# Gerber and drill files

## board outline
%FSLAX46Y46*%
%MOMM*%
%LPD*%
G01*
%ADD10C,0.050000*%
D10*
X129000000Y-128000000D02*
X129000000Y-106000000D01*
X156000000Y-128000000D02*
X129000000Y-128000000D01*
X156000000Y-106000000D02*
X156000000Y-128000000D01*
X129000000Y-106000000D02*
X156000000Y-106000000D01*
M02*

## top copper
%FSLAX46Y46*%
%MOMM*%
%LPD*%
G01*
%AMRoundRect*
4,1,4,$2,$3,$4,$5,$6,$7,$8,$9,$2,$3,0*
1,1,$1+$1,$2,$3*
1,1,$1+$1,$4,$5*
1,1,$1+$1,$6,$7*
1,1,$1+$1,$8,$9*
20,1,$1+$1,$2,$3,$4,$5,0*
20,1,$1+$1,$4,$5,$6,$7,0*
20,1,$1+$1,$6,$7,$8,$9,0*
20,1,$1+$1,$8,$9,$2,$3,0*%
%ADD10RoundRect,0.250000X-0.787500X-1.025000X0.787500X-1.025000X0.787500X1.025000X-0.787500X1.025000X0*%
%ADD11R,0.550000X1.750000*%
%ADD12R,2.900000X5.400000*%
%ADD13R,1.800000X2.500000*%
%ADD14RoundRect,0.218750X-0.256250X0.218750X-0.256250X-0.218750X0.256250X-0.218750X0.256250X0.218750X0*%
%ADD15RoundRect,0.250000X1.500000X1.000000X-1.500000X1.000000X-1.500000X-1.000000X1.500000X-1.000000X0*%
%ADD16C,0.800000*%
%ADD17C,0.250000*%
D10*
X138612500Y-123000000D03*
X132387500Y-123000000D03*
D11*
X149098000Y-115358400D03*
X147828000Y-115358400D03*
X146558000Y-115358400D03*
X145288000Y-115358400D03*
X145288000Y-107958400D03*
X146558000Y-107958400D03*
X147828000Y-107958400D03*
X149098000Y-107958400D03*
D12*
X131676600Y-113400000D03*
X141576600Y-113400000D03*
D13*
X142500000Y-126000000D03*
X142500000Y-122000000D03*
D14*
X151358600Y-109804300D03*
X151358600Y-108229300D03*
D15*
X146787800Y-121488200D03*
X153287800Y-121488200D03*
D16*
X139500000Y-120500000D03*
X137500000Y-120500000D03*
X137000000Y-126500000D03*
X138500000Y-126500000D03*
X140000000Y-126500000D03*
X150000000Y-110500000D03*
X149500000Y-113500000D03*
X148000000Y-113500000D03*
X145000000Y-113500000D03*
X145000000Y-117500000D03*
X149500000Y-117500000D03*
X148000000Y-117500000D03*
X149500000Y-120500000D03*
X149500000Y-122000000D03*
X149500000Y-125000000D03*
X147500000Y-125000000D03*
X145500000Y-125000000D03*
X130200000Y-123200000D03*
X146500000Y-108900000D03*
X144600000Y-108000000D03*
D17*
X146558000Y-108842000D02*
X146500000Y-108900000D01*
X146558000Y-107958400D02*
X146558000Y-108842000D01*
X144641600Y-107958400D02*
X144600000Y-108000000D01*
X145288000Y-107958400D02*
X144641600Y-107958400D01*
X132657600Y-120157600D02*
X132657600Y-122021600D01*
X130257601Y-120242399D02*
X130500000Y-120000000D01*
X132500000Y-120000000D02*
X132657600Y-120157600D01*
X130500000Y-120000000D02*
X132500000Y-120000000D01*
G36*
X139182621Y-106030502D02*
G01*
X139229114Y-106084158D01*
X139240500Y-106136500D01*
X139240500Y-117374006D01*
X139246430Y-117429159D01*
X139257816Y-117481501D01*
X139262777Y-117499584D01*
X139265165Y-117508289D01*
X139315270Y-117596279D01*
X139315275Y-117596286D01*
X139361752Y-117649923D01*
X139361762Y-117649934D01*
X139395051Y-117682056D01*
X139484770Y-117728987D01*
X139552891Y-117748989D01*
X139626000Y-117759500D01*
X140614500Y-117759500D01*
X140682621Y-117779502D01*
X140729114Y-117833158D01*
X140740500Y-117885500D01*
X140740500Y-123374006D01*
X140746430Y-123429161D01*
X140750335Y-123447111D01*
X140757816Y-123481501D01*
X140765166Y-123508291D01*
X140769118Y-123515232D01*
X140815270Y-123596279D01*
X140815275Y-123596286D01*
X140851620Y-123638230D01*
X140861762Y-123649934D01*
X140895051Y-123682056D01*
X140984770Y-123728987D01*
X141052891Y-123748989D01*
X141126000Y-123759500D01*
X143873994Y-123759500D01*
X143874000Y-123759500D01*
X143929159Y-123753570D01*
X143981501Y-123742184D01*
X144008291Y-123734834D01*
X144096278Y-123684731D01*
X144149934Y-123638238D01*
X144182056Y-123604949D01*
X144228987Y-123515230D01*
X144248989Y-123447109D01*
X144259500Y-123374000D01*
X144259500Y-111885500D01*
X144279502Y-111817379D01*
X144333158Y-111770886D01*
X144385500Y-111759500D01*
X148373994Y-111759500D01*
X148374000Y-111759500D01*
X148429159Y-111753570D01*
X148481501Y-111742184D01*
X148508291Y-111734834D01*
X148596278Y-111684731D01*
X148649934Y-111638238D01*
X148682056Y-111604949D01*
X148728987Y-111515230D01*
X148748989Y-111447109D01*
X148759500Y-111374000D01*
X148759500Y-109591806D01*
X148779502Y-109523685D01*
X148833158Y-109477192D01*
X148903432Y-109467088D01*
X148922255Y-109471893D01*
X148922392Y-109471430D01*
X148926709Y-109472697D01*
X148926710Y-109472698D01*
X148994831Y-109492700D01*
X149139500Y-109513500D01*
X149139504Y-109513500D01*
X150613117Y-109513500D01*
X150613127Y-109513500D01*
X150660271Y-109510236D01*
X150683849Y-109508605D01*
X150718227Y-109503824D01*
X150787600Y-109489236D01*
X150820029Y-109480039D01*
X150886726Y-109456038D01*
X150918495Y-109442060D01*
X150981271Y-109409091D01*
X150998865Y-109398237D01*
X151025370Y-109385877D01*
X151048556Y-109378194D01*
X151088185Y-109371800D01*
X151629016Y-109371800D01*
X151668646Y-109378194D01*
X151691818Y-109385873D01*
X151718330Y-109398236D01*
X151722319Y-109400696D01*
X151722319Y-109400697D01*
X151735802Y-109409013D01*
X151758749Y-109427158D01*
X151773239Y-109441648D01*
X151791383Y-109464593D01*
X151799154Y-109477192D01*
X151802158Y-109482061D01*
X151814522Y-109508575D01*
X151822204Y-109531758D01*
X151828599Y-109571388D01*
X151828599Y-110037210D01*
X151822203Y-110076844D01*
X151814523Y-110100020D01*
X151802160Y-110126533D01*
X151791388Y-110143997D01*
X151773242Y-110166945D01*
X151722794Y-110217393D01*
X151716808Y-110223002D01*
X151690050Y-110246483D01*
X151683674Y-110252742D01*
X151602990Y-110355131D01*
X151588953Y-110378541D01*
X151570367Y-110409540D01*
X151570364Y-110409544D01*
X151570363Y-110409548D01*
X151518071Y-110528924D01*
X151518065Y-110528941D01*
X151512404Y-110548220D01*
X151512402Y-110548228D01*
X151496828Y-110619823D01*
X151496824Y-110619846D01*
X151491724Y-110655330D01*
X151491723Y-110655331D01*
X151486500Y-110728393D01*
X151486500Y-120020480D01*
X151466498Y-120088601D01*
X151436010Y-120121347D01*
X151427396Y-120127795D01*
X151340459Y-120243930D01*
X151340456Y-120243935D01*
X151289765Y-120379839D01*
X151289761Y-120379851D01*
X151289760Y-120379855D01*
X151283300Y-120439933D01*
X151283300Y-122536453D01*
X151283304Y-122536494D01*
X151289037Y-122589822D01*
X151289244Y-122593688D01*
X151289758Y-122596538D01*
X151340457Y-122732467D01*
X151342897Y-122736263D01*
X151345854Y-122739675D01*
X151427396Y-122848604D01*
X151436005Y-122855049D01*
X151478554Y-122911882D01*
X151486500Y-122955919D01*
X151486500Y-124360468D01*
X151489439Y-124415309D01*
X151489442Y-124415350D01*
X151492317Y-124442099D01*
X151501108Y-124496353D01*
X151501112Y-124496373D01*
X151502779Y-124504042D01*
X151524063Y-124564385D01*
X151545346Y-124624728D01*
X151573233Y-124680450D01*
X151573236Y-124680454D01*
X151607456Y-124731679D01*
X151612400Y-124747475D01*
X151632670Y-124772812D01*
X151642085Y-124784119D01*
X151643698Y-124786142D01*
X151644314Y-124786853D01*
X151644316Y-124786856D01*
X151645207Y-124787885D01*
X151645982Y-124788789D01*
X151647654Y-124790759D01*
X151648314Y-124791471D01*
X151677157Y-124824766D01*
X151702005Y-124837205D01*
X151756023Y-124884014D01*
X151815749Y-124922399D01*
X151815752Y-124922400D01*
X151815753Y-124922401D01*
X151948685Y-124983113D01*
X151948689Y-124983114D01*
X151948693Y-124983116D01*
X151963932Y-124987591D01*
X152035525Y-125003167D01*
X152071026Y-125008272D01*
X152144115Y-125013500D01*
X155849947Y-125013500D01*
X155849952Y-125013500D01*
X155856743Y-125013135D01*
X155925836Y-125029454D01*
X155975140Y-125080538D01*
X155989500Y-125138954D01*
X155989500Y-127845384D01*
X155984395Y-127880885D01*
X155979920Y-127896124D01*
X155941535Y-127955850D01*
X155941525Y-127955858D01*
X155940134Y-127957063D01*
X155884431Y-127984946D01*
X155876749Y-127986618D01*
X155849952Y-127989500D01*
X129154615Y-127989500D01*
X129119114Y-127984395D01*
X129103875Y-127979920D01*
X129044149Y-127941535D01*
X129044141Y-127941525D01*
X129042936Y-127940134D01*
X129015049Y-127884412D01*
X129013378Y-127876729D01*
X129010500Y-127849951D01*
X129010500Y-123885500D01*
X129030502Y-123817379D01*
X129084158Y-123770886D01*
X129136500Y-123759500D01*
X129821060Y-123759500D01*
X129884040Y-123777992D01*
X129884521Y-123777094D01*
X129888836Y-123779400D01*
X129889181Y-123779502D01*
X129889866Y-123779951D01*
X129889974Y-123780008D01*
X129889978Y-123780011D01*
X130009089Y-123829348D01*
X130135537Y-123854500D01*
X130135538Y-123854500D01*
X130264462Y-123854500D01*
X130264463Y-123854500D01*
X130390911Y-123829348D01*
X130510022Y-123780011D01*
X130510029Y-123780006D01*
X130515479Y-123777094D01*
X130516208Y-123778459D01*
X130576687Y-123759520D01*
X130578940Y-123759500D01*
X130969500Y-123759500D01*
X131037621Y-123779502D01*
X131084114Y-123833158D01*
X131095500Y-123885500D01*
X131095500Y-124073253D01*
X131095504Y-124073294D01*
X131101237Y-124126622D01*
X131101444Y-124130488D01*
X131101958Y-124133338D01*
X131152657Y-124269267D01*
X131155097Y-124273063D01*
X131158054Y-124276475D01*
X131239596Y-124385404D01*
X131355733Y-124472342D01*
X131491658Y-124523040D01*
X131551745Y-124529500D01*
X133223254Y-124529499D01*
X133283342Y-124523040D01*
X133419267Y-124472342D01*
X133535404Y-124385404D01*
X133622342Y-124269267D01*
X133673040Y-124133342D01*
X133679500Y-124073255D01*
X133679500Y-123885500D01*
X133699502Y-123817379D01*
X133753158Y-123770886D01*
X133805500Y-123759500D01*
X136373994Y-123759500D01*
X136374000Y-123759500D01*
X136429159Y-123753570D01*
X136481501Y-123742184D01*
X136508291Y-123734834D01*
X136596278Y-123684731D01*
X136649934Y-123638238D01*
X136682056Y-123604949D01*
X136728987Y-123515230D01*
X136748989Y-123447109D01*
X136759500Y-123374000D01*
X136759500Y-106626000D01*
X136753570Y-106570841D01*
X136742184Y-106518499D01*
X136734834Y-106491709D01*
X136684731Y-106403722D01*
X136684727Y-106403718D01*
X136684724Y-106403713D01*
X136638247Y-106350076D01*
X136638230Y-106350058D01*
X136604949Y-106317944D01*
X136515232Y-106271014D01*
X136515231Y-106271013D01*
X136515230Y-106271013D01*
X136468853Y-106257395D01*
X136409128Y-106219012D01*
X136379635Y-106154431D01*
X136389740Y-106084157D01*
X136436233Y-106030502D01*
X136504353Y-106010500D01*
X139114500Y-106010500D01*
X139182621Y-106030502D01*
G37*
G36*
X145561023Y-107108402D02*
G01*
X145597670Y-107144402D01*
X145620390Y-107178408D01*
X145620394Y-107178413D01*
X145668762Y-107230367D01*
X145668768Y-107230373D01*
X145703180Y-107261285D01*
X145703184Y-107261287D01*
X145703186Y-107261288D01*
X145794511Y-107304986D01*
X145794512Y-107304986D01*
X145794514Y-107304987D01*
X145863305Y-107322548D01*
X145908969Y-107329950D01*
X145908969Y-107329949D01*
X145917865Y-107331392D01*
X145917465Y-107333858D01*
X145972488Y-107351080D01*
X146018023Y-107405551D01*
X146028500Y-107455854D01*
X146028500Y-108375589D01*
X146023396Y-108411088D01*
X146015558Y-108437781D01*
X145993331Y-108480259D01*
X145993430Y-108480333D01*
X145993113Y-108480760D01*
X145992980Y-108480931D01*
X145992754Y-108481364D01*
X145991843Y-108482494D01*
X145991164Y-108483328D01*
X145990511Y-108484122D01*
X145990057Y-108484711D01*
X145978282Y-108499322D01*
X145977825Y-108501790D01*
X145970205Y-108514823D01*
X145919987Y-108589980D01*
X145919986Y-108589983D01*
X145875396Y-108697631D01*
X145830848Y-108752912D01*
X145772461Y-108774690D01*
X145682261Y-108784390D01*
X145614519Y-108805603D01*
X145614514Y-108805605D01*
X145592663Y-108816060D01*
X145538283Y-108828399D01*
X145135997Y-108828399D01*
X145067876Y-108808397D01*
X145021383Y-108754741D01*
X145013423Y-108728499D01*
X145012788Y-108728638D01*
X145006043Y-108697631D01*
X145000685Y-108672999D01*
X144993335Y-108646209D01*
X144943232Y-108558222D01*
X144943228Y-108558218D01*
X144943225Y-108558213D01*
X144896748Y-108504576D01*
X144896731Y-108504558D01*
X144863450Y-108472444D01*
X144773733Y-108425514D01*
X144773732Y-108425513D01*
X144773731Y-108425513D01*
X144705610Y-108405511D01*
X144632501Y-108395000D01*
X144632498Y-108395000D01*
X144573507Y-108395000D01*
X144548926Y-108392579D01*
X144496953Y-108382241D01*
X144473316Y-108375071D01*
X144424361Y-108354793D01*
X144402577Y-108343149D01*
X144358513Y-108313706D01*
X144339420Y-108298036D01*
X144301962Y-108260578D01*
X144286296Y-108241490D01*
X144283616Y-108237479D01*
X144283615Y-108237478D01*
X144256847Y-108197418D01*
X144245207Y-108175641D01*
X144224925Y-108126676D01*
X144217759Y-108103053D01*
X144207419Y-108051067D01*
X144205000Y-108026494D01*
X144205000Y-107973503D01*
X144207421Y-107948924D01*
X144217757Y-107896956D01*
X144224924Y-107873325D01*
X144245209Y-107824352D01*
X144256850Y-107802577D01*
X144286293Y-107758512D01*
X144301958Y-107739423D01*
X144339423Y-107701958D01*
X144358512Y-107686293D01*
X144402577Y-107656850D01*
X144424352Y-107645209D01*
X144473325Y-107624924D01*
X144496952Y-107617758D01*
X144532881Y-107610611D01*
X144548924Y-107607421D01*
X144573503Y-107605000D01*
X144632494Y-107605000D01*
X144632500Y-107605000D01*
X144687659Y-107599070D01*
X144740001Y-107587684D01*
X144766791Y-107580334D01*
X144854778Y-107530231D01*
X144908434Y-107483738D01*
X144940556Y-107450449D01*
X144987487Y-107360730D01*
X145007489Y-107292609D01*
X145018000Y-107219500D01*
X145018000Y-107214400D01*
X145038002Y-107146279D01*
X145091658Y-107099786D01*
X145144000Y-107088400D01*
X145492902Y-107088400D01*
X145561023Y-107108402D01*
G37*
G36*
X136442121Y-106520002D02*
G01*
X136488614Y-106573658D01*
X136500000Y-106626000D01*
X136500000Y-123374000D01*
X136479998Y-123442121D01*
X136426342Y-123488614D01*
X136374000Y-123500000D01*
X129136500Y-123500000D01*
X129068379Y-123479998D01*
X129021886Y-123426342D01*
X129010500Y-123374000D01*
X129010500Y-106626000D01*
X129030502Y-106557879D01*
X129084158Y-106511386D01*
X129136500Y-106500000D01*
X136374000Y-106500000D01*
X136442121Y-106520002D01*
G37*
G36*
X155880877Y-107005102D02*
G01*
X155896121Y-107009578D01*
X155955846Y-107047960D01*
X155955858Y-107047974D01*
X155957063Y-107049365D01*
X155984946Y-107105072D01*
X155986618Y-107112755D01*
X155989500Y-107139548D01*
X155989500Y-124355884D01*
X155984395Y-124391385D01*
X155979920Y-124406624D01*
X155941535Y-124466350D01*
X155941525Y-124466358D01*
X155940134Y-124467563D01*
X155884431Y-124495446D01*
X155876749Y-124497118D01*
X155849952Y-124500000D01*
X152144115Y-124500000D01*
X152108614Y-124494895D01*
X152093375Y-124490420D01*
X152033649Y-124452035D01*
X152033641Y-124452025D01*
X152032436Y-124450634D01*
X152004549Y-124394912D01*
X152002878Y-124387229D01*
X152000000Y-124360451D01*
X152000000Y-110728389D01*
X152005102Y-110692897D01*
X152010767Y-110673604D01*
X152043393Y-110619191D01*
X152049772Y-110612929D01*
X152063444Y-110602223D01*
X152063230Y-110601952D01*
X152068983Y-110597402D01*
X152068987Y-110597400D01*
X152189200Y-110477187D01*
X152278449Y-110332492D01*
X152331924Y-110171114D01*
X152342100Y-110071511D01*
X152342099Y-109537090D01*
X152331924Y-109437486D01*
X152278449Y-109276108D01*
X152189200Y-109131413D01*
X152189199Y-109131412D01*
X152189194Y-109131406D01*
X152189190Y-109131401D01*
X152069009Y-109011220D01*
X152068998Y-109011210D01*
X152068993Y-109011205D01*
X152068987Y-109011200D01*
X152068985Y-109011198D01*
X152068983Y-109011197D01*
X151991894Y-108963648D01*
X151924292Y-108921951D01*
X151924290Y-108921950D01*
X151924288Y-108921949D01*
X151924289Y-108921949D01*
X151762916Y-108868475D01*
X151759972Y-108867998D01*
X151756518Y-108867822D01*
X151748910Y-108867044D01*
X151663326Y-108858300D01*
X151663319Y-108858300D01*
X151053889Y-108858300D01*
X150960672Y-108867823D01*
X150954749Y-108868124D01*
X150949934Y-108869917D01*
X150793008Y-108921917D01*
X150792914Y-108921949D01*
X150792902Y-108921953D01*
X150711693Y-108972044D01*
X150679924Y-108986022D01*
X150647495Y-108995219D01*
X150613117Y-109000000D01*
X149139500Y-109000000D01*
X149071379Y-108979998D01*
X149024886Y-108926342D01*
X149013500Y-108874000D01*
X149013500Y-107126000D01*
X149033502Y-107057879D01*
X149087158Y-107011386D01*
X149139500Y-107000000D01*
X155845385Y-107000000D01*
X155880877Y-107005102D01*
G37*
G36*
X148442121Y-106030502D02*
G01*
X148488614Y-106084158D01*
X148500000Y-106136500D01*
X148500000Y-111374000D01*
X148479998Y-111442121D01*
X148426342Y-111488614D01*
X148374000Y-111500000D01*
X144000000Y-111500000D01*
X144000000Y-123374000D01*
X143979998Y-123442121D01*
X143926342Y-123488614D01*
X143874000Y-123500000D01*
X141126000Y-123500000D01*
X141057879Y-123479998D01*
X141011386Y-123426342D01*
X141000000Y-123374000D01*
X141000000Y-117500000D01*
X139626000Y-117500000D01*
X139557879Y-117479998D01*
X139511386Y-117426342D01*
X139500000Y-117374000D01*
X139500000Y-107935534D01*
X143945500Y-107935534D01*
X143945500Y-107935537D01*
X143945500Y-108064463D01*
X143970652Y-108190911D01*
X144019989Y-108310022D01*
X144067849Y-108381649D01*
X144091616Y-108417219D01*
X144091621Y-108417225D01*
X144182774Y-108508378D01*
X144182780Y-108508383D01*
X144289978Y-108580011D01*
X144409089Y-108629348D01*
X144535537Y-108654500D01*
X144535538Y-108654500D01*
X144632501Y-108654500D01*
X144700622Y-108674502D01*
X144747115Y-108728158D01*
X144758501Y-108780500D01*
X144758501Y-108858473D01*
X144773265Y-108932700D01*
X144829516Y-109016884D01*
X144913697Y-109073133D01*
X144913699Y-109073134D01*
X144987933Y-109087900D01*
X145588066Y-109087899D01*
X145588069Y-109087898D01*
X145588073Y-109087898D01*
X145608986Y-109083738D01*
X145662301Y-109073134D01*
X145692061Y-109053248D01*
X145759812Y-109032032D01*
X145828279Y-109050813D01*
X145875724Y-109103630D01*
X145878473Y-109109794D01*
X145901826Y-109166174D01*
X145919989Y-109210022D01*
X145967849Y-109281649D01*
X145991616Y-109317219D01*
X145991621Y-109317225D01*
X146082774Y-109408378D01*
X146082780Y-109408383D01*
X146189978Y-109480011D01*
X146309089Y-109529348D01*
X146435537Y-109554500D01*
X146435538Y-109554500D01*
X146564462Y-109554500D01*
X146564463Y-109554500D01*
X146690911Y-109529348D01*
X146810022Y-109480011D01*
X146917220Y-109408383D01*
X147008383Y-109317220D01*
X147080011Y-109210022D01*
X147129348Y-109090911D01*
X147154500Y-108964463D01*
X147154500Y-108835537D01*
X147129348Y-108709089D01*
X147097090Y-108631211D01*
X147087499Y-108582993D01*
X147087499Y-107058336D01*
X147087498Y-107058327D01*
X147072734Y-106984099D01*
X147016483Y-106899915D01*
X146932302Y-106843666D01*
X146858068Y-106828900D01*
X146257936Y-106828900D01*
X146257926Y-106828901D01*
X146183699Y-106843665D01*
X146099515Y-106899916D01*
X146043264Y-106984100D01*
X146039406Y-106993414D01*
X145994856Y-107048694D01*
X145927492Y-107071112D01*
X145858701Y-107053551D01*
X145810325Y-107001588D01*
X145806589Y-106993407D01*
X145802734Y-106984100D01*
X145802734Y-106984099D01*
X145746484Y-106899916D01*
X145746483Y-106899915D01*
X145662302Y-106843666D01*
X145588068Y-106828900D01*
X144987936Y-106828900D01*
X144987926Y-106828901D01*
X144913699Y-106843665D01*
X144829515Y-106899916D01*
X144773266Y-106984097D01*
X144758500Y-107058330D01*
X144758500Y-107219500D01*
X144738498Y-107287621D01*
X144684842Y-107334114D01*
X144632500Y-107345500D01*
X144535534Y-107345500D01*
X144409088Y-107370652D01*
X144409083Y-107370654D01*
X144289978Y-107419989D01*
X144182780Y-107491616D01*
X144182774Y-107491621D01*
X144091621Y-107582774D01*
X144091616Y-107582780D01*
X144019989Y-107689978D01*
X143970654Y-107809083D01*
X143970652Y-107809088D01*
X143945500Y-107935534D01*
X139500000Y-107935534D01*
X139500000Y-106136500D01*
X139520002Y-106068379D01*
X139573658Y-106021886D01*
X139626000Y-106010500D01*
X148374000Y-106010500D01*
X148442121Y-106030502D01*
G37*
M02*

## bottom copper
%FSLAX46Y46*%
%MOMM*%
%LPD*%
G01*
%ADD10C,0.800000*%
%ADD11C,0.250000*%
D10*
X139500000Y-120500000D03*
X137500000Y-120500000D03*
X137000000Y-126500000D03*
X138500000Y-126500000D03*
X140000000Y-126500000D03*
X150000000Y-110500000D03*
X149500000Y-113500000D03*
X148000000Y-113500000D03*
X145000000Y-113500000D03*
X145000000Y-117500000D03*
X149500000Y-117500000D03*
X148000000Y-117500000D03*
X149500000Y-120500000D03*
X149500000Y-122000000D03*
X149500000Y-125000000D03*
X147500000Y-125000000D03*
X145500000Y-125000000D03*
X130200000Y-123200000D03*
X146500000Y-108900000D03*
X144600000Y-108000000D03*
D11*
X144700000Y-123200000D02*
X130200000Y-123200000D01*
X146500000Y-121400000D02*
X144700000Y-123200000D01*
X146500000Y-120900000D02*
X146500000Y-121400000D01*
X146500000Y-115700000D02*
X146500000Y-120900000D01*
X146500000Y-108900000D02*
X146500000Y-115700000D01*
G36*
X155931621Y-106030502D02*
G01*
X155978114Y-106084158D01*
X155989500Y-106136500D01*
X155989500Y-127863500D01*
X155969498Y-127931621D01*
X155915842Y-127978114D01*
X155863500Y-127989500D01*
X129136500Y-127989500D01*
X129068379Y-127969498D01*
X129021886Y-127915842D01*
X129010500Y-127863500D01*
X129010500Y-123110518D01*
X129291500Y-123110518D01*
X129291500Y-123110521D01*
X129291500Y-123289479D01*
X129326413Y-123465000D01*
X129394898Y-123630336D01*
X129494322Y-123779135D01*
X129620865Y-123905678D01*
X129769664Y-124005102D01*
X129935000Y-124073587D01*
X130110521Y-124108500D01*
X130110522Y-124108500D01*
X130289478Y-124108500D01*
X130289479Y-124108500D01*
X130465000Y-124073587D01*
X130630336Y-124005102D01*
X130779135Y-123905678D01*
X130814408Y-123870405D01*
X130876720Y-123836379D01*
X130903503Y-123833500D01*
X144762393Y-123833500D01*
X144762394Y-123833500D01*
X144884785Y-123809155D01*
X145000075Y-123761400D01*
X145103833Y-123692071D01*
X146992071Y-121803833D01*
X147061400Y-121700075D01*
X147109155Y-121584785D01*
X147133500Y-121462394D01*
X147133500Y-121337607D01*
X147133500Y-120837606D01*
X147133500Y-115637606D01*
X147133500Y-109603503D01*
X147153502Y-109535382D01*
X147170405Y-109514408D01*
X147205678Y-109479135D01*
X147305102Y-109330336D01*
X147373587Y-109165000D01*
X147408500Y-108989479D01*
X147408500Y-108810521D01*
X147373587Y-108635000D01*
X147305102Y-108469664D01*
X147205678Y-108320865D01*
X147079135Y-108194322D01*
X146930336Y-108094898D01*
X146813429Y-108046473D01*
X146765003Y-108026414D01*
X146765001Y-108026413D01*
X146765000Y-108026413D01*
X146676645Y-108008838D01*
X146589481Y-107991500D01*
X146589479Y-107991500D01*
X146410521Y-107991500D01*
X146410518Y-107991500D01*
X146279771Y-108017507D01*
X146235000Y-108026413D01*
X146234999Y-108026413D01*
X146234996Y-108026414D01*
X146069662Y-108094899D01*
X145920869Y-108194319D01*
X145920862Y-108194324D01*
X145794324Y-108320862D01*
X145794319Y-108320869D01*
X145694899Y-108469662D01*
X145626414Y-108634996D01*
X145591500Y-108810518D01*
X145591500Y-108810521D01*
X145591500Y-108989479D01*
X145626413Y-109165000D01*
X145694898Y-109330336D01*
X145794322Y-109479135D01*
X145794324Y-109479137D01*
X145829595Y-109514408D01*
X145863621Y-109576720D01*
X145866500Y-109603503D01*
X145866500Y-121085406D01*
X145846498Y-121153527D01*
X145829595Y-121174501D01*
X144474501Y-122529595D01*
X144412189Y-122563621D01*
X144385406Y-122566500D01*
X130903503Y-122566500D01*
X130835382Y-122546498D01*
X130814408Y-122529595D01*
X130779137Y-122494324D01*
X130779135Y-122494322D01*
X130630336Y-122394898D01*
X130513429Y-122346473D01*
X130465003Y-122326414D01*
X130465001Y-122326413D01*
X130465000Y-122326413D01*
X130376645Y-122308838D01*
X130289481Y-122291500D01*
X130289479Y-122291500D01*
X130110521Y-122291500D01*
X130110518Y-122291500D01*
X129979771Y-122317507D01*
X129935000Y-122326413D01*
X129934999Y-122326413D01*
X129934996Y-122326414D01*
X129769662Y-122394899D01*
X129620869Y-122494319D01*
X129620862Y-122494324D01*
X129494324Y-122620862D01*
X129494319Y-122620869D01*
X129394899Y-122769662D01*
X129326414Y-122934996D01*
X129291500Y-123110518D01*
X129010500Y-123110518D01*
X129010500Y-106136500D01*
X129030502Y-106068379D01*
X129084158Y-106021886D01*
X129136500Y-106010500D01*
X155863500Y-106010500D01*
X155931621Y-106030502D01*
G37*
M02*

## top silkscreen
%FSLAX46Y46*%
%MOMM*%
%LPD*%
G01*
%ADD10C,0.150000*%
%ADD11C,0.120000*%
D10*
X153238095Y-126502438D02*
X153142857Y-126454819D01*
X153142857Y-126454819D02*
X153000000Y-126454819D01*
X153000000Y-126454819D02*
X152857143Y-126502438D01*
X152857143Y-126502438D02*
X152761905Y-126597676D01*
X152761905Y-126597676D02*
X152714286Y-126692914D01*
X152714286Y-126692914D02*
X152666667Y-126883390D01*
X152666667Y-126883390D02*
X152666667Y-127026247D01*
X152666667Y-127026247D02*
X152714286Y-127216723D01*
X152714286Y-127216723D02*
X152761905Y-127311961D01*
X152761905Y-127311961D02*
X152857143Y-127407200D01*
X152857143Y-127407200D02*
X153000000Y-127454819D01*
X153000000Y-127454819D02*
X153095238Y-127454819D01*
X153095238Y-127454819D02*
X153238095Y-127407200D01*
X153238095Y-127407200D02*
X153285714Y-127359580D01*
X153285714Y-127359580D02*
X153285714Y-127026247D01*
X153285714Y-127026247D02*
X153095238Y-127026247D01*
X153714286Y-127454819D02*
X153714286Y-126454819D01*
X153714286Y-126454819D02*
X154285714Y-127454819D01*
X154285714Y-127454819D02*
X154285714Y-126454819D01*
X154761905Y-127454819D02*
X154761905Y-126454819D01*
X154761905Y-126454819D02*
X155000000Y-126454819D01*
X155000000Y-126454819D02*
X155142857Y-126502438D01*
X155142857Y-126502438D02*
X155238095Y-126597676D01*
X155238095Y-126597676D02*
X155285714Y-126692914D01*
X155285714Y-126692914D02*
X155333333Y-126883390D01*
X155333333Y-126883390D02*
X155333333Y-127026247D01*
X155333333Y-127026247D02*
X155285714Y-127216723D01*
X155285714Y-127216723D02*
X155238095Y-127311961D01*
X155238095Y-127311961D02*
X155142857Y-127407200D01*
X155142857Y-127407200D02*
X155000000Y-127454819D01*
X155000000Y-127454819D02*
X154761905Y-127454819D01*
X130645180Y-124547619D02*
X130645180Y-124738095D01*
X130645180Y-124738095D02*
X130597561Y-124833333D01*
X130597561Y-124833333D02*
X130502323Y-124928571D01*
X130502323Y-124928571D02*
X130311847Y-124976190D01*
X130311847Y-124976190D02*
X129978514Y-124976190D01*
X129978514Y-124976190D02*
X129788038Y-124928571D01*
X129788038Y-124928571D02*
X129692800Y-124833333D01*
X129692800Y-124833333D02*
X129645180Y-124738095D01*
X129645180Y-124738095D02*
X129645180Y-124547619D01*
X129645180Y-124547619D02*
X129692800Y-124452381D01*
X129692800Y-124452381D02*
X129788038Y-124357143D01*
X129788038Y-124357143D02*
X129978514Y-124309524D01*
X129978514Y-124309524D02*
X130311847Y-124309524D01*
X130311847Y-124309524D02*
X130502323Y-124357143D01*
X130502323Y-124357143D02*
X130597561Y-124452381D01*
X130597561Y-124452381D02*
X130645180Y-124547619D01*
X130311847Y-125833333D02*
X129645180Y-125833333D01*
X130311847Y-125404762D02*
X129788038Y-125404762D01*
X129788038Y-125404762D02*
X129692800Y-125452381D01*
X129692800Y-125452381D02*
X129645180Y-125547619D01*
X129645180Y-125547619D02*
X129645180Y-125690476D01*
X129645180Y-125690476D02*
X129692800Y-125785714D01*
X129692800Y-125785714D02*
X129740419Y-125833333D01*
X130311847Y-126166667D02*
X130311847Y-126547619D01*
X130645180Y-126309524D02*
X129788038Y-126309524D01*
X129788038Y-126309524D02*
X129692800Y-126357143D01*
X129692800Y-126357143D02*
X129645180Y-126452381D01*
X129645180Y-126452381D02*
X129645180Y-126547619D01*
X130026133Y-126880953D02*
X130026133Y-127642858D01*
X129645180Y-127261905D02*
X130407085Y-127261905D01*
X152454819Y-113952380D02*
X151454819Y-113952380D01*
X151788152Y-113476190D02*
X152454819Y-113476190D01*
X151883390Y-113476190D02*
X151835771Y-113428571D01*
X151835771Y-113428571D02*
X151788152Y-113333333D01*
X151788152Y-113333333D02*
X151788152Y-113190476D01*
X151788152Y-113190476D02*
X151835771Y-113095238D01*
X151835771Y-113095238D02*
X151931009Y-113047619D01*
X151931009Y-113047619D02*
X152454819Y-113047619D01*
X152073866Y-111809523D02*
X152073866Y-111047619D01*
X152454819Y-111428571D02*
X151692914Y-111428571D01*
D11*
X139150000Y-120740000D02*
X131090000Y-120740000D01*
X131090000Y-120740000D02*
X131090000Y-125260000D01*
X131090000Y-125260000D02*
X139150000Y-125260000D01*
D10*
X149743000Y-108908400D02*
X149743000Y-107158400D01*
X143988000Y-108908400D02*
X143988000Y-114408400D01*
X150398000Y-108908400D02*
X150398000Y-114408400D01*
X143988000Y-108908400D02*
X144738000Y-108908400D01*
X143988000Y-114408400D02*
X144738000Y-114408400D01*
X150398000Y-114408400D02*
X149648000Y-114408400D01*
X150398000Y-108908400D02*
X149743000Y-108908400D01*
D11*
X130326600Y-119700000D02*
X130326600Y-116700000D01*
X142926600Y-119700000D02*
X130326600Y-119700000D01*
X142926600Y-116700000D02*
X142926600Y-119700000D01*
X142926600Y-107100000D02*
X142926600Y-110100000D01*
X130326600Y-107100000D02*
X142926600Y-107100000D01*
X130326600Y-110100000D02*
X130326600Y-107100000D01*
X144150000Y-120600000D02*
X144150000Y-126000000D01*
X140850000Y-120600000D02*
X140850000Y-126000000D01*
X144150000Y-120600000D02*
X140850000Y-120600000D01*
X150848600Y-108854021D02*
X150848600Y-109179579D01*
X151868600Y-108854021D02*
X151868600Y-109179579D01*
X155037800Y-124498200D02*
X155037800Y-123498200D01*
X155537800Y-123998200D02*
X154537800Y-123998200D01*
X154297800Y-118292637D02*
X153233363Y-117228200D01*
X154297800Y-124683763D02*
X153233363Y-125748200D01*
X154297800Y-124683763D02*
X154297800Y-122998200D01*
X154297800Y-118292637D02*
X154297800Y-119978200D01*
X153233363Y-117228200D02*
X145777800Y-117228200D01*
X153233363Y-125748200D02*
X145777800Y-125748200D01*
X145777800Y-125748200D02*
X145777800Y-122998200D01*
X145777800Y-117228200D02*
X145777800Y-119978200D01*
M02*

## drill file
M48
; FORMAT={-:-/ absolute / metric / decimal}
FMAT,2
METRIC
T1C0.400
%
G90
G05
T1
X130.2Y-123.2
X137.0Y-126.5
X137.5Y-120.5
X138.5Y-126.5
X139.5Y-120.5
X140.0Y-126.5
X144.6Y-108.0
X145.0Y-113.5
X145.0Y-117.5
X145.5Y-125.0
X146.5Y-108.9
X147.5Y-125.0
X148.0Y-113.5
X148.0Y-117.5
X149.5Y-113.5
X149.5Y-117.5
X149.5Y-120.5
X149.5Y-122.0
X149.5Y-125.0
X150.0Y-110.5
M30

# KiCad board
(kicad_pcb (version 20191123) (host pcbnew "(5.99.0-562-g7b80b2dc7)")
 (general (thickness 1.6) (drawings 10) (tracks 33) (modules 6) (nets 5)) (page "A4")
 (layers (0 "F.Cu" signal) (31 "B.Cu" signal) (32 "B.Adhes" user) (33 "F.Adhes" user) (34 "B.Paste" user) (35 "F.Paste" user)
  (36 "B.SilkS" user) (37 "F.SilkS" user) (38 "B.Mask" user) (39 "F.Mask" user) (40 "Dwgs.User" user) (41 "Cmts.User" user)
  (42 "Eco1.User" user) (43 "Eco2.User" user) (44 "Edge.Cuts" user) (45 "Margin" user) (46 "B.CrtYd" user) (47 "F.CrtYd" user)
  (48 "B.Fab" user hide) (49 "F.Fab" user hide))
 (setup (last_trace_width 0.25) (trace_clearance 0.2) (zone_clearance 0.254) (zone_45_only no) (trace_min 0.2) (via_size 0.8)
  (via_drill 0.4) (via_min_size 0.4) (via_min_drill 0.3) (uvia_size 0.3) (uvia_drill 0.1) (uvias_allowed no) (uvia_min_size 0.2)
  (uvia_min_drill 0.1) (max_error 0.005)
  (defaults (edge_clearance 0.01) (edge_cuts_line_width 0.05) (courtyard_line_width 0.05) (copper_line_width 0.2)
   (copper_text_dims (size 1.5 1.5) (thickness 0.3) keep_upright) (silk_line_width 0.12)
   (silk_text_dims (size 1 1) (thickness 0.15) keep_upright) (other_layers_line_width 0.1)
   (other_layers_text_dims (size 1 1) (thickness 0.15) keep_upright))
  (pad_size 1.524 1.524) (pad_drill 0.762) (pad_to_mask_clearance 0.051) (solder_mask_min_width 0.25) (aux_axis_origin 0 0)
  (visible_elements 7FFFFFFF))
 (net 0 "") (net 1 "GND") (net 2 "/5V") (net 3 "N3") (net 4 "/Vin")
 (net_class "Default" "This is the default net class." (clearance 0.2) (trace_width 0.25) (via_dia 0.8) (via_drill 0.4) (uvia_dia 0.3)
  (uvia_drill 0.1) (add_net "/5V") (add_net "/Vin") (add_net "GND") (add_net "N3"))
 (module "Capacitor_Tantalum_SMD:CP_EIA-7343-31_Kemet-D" (layer "F.Cu") (at 135.5 123)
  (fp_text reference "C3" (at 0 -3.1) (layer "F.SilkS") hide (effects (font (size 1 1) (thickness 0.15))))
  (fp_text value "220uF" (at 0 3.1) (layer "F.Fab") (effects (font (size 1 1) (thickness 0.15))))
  (fp_line (start 3.65 -2.26) (end -4.41 -2.26) (layer "F.SilkS") (width 0.12))
  (fp_line (start -4.41 -2.26) (end -4.41 2.26) (layer "F.SilkS") (width 0.12))
  (fp_line (start -4.41 2.26) (end 3.65 2.26) (layer "F.SilkS") (width 0.12))
  (pad "2" smd roundrect (at 3.1125 0) (size 2.075 2.55) (layers "F.Cu" "F.Paste" "F.Mask") (roundrect_rratio 0.120482) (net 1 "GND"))
  (pad "1" smd roundrect (at -3.1125 0) (size 2.075 2.55) (layers "F.Cu" "F.Paste" "F.Mask") (roundrect_rratio 0.120482) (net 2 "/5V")))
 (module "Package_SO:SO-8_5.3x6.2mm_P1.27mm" (layer "F.Cu") (at 147.193 111.6584 -90)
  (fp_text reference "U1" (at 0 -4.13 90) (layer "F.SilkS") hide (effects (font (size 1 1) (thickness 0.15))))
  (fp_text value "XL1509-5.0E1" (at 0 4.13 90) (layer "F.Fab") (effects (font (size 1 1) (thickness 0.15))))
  (fp_line (start -2.75 -2.55) (end -4.5 -2.55) (layer "F.SilkS") (width 0.15))
  (fp_line (start -2.75 3.205) (end 2.75 3.205) (layer "F.SilkS") (width 0.15))
  (fp_line (start -2.75 -3.205) (end 2.75 -3.205) (layer "F.SilkS") (width 0.15))
  (fp_line (start -2.75 3.205) (end -2.75 2.455) (layer "F.SilkS") (width 0.15))
  (fp_line (start 2.75 3.205) (end 2.75 2.455) (layer "F.SilkS") (width 0.15))
  (fp_line (start 2.75 -3.205) (end 2.75 -2.455) (layer "F.SilkS") (width 0.15))
  (fp_line (start -2.75 -3.205) (end -2.75 -2.55) (layer "F.SilkS") (width 0.15))
  (pad "8" smd rect (at 3.7 -1.905 270) (size 1.75 0.55) (layers "F.Cu" "F.Paste" "F.Mask") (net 1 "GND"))
  (pad "7" smd rect (at 3.7 -0.635 270) (size 1.75 0.55) (layers "F.Cu" "F.Paste" "F.Mask") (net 1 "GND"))
  (pad "6" smd rect (at 3.7 0.635 270) (size 1.75 0.55) (layers "F.Cu" "F.Paste" "F.Mask") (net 1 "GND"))
  (pad "5" smd rect (at 3.7 1.905 270) (size 1.75 0.55) (layers "F.Cu" "F.Paste" "F.Mask") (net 1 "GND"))
  (pad "4" smd rect (at -3.7 1.905 270) (size 1.75 0.55) (layers "F.Cu" "F.Paste" "F.Mask") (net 1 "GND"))
  (pad "3" smd rect (at -3.7 0.635 270) (size 1.75 0.55) (layers "F.Cu" "F.Paste" "F.Mask") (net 2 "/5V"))
  (pad "2" smd rect (at -3.7 -0.635 270) (size 1.75 0.55) (layers "F.Cu" "F.Paste" "F.Mask") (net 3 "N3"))
  (pad "1" smd rect (at -3.7 -1.905 270) (size 1.75 0.55) (layers "F.Cu" "F.Paste" "F.Mask") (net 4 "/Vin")))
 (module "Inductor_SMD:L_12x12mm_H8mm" (layer "F.Cu") (at 136.6266 113.4 180)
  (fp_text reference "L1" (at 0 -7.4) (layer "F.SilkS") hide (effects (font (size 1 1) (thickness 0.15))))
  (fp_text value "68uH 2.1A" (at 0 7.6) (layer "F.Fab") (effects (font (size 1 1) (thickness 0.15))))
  (fp_line (start 6.3 -6.3) (end 6.3 -3.3) (layer "F.SilkS") (width 0.12))
  (fp_line (start -6.3 -6.3) (end 6.3 -6.3) (layer "F.SilkS") (width 0.12))
  (fp_line (start -6.3 -3.3) (end -6.3 -6.3) (layer "F.SilkS") (width 0.12))
  (fp_line (start -6.3 6.3) (end -6.3 3.3) (layer "F.SilkS") (width 0.12))
  (fp_line (start 6.3 6.3) (end -6.3 6.3) (layer "F.SilkS") (width 0.12))
  (fp_line (start 6.3 3.3) (end 6.3 6.3) (layer "F.SilkS") (width 0.12))
  (pad "2" smd rect (at 4.95 0 180) (size 2.9 5.4) (layers "F.Cu" "F.Paste" "F.Mask") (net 2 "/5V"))
  (pad "1" smd rect (at -4.95 0 180) (size 2.9 5.4) (layers "F.Cu" "F.Paste" "F.Mask") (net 3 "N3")))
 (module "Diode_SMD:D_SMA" (layer "F.Cu") (at 142.5 124 -90)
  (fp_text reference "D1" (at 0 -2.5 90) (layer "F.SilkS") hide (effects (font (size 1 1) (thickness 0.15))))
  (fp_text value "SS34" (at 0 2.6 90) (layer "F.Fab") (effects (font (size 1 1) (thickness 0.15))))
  (fp_line (start -3.4 -1.65) (end 2 -1.65) (layer "F.SilkS") (width 0.12))
  (fp_line (start -3.4 1.65) (end 2 1.65) (layer "F.SilkS") (width 0.12))
  (fp_line (start -3.4 -1.65) (end -3.4 1.65) (layer "F.SilkS") (width 0.12))
  (pad "2" smd rect (at 2 0 270) (size 2.5 1.8) (layers "F.Cu" "F.Paste" "F.Mask") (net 1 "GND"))
  (pad "1" smd rect (at -2 0 270) (size 2.5 1.8) (layers "F.Cu" "F.Paste" "F.Mask") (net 3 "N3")))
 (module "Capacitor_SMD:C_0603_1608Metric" (layer "F.Cu") (at 151.3586 109.0168 -90)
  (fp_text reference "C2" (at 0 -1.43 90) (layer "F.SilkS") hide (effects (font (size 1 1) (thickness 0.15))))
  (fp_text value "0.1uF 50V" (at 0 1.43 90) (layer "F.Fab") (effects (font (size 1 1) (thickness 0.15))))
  (fp_line (start -0.162779 0.51) (end 0.162779 0.51) (layer "F.SilkS") (width 0.12))
  (fp_line (start -0.162779 -0.51) (end 0.162779 -0.51) (layer "F.SilkS") (width 0.12))
  (pad "2" smd roundrect (at 0.7875 0 270) (size 0.875 0.95) (layers "F.Cu" "F.Paste" "F.Mask") (roundrect_rratio 0.25) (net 1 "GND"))
  (pad "1" smd roundrect (at -0.7875 0 270) (size 0.875 0.95) (layers "F.Cu" "F.Paste" "F.Mask") (roundrect_rratio 0.25) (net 4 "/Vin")))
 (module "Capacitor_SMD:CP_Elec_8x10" (layer "F.Cu") (at 150.0378 121.4882 180)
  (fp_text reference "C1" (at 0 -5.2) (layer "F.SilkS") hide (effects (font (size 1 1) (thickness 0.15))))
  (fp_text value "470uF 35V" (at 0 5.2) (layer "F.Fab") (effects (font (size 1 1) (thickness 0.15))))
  (fp_line (start -5 -3.01) (end -5 -2.01) (layer "F.SilkS") (width 0.12))
  (fp_line (start -5.5 -2.51) (end -4.5 -2.51) (layer "F.SilkS") (width 0.12))
  (fp_line (start -4.26 3.195563) (end -3.195563 4.26) (layer "F.SilkS") (width 0.12))
  (fp_line (start -4.26 -3.195563) (end -3.195563 -4.26) (layer "F.SilkS") (width 0.12))
  (fp_line (start -4.26 -3.195563) (end -4.26 -1.51) (layer "F.SilkS") (width 0.12))
  (fp_line (start -4.26 3.195563) (end -4.26 1.51) (layer "F.SilkS") (width 0.12))
  (fp_line (start -3.195563 4.26) (end 4.26 4.26) (layer "F.SilkS") (width 0.12))
  (fp_line (start -3.195563 -4.26) (end 4.26 -4.26) (layer "F.SilkS") (width 0.12))
  (fp_line (start 4.26 -4.26) (end 4.26 -1.51) (layer "F.SilkS") (width 0.12))
  (fp_line (start 4.26 4.26) (end 4.26 1.51) (layer "F.SilkS") (width 0.12))
  (pad "2" smd roundrect (at 3.25 0 180) (size 3.5 2.5) (layers "F.Cu" "F.Paste" "F.Mask") (roundrect_rratio 0.1) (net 1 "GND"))
  (pad "1" smd roundrect (at -3.25 0 180) (size 3.5 2.5) (layers "F.Cu" "F.Paste" "F.Mask") (roundrect_rratio 0.1) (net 4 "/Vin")))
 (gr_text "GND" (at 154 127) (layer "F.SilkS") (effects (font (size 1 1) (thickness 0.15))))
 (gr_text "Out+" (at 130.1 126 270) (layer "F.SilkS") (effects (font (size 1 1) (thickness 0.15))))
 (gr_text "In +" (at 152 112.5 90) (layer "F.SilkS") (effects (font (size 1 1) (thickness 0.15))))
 (gr_line (start 129 128) (end 129 106) (layer "Edge.Cuts") (width 0.05))
 (gr_line (start 156 128) (end 129 128) (layer "Edge.Cuts") (width 0.05))
 (gr_line (start 156 106) (end 156 128) (layer "Edge.Cuts") (width 0.05))
 (gr_line (start 129 106) (end 156 106) (layer "Edge.Cuts") (width 0.05))
 (via (at 139.5 120.5) (size 0.8) (drill 0.4) (layers "F.Cu" "B.Cu") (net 1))
 (via (at 137.5 120.5) (size 0.8) (drill 0.4) (layers "F.Cu" "B.Cu") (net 1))
 (via (at 137 126.5) (size 0.8) (drill 0.4) (layers "F.Cu" "B.Cu") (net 1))
 (via (at 138.5 126.5) (size 0.8) (drill 0.4) (layers "F.Cu" "B.Cu") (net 1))
 (via (at 140 126.5) (size 0.8) (drill 0.4) (layers "F.Cu" "B.Cu") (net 1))
 (via (at 150 110.5) (size 0.8) (drill 0.4) (layers "F.Cu" "B.Cu") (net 1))
 (via (at 149.5 113.5) (size 0.8) (drill 0.4) (layers "F.Cu" "B.Cu") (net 1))
 (via (at 148 113.5) (size 0.8) (drill 0.4) (layers "F.Cu" "B.Cu") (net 1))
 (via (at 145 113.5) (size 0.8) (drill 0.4) (layers "F.Cu" "B.Cu") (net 1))
 (via (at 145 117.5) (size 0.8) (drill 0.4) (layers "F.Cu" "B.Cu") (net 1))
 (via (at 149.5 117.5) (size 0.8) (drill 0.4) (layers "F.Cu" "B.Cu") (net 1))
 (via (at 148 117.5) (size 0.8) (drill 0.4) (layers "F.Cu" "B.Cu") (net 1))
 (via (at 149.5 120.5) (size 0.8) (drill 0.4) (layers "F.Cu" "B.Cu") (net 1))
 (via (at 149.5 122) (size 0.8) (drill 0.4) (layers "F.Cu" "B.Cu") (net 1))
 (via (at 149.5 125) (size 0.8) (drill 0.4) (layers "F.Cu" "B.Cu") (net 1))
 (via (at 147.5 125) (size 0.8) (drill 0.4) (layers "F.Cu" "B.Cu") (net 1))
 (via (at 145.5 125) (size 0.8) (drill 0.4) (layers "F.Cu" "B.Cu") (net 1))
 (segment (start 144.7 123.2) (end 130.2 123.2) (width 0.25) (layer "B.Cu") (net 2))
 (segment (start 146.5 121.4) (end 144.7 123.2) (width 0.25) (layer "B.Cu") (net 2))
 (via (at 130.2 123.2) (size 0.8) (drill 0.4) (layers "F.Cu" "B.Cu") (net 2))
 (segment (start 146.5 120.9) (end 146.5 121.4) (width 0.25) (layer "B.Cu") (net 2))
 (segment (start 146.5 115.7) (end 146.5 120.9) (width 0.25) (layer "B.Cu") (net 2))
 (segment (start 146.5 108.9) (end 146.5 115.7) (width 0.25) (layer "B.Cu") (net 2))
 (segment (start 146.558 108.842) (end 146.5 108.9) (width 0.25) (layer "F.Cu") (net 2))
 (segment (start 146.558 107.9584) (end 146.558 108.842) (width 0.25) (layer "F.Cu") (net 2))
 (via (at 146.5 108.9) (size 0.8) (drill 0.4) (layers "F.Cu" "B.Cu") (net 2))
 (segment (start 144.6416 107.9584) (end 144.6 108) (width 0.25) (layer "F.Cu") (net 1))
 (via (at 144.6 108) (size 0.8) (drill 0.4) (layers "F.Cu" "B.Cu") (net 1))
 (segment (start 145.288 107.9584) (end 144.6416 107.9584) (width 0.25) (layer "F.Cu") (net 1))
 (segment (start 132.6576 120.1576) (end 132.6576 122.0216) (width 0.25) (layer "F.Cu") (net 2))
 (segment (start 130.257601 120.242399) (end 130.5 120) (width 0.25) (layer "F.Cu") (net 2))
 (segment (start 132.5 120) (end 132.6576 120.1576) (width 0.25) (layer "F.Cu") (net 2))
 (segment (start 130.5 120) (end 132.5 120) (width 0.25) (layer "F.Cu") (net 2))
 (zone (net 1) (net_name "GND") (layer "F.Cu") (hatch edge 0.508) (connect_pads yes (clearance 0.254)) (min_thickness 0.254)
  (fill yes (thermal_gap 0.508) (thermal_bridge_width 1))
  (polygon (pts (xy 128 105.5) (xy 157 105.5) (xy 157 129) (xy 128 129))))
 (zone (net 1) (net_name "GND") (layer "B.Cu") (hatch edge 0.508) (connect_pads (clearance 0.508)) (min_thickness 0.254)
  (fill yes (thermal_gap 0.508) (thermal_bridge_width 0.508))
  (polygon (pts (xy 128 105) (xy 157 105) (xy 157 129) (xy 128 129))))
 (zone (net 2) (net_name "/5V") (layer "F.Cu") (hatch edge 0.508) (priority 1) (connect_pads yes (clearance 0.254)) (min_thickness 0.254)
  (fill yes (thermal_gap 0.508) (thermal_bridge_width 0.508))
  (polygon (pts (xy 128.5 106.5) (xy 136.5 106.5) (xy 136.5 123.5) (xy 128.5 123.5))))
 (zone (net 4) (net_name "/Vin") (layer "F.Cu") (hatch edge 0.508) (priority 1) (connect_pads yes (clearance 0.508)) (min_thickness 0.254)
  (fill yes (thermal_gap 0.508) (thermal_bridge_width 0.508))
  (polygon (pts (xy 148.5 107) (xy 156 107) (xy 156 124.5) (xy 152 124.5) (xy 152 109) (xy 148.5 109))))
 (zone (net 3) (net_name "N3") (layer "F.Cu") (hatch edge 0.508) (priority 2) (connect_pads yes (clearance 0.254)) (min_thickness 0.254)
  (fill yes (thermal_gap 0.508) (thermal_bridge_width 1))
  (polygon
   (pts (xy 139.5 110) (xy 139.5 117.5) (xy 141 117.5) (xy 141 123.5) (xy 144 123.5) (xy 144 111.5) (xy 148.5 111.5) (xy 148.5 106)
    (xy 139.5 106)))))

